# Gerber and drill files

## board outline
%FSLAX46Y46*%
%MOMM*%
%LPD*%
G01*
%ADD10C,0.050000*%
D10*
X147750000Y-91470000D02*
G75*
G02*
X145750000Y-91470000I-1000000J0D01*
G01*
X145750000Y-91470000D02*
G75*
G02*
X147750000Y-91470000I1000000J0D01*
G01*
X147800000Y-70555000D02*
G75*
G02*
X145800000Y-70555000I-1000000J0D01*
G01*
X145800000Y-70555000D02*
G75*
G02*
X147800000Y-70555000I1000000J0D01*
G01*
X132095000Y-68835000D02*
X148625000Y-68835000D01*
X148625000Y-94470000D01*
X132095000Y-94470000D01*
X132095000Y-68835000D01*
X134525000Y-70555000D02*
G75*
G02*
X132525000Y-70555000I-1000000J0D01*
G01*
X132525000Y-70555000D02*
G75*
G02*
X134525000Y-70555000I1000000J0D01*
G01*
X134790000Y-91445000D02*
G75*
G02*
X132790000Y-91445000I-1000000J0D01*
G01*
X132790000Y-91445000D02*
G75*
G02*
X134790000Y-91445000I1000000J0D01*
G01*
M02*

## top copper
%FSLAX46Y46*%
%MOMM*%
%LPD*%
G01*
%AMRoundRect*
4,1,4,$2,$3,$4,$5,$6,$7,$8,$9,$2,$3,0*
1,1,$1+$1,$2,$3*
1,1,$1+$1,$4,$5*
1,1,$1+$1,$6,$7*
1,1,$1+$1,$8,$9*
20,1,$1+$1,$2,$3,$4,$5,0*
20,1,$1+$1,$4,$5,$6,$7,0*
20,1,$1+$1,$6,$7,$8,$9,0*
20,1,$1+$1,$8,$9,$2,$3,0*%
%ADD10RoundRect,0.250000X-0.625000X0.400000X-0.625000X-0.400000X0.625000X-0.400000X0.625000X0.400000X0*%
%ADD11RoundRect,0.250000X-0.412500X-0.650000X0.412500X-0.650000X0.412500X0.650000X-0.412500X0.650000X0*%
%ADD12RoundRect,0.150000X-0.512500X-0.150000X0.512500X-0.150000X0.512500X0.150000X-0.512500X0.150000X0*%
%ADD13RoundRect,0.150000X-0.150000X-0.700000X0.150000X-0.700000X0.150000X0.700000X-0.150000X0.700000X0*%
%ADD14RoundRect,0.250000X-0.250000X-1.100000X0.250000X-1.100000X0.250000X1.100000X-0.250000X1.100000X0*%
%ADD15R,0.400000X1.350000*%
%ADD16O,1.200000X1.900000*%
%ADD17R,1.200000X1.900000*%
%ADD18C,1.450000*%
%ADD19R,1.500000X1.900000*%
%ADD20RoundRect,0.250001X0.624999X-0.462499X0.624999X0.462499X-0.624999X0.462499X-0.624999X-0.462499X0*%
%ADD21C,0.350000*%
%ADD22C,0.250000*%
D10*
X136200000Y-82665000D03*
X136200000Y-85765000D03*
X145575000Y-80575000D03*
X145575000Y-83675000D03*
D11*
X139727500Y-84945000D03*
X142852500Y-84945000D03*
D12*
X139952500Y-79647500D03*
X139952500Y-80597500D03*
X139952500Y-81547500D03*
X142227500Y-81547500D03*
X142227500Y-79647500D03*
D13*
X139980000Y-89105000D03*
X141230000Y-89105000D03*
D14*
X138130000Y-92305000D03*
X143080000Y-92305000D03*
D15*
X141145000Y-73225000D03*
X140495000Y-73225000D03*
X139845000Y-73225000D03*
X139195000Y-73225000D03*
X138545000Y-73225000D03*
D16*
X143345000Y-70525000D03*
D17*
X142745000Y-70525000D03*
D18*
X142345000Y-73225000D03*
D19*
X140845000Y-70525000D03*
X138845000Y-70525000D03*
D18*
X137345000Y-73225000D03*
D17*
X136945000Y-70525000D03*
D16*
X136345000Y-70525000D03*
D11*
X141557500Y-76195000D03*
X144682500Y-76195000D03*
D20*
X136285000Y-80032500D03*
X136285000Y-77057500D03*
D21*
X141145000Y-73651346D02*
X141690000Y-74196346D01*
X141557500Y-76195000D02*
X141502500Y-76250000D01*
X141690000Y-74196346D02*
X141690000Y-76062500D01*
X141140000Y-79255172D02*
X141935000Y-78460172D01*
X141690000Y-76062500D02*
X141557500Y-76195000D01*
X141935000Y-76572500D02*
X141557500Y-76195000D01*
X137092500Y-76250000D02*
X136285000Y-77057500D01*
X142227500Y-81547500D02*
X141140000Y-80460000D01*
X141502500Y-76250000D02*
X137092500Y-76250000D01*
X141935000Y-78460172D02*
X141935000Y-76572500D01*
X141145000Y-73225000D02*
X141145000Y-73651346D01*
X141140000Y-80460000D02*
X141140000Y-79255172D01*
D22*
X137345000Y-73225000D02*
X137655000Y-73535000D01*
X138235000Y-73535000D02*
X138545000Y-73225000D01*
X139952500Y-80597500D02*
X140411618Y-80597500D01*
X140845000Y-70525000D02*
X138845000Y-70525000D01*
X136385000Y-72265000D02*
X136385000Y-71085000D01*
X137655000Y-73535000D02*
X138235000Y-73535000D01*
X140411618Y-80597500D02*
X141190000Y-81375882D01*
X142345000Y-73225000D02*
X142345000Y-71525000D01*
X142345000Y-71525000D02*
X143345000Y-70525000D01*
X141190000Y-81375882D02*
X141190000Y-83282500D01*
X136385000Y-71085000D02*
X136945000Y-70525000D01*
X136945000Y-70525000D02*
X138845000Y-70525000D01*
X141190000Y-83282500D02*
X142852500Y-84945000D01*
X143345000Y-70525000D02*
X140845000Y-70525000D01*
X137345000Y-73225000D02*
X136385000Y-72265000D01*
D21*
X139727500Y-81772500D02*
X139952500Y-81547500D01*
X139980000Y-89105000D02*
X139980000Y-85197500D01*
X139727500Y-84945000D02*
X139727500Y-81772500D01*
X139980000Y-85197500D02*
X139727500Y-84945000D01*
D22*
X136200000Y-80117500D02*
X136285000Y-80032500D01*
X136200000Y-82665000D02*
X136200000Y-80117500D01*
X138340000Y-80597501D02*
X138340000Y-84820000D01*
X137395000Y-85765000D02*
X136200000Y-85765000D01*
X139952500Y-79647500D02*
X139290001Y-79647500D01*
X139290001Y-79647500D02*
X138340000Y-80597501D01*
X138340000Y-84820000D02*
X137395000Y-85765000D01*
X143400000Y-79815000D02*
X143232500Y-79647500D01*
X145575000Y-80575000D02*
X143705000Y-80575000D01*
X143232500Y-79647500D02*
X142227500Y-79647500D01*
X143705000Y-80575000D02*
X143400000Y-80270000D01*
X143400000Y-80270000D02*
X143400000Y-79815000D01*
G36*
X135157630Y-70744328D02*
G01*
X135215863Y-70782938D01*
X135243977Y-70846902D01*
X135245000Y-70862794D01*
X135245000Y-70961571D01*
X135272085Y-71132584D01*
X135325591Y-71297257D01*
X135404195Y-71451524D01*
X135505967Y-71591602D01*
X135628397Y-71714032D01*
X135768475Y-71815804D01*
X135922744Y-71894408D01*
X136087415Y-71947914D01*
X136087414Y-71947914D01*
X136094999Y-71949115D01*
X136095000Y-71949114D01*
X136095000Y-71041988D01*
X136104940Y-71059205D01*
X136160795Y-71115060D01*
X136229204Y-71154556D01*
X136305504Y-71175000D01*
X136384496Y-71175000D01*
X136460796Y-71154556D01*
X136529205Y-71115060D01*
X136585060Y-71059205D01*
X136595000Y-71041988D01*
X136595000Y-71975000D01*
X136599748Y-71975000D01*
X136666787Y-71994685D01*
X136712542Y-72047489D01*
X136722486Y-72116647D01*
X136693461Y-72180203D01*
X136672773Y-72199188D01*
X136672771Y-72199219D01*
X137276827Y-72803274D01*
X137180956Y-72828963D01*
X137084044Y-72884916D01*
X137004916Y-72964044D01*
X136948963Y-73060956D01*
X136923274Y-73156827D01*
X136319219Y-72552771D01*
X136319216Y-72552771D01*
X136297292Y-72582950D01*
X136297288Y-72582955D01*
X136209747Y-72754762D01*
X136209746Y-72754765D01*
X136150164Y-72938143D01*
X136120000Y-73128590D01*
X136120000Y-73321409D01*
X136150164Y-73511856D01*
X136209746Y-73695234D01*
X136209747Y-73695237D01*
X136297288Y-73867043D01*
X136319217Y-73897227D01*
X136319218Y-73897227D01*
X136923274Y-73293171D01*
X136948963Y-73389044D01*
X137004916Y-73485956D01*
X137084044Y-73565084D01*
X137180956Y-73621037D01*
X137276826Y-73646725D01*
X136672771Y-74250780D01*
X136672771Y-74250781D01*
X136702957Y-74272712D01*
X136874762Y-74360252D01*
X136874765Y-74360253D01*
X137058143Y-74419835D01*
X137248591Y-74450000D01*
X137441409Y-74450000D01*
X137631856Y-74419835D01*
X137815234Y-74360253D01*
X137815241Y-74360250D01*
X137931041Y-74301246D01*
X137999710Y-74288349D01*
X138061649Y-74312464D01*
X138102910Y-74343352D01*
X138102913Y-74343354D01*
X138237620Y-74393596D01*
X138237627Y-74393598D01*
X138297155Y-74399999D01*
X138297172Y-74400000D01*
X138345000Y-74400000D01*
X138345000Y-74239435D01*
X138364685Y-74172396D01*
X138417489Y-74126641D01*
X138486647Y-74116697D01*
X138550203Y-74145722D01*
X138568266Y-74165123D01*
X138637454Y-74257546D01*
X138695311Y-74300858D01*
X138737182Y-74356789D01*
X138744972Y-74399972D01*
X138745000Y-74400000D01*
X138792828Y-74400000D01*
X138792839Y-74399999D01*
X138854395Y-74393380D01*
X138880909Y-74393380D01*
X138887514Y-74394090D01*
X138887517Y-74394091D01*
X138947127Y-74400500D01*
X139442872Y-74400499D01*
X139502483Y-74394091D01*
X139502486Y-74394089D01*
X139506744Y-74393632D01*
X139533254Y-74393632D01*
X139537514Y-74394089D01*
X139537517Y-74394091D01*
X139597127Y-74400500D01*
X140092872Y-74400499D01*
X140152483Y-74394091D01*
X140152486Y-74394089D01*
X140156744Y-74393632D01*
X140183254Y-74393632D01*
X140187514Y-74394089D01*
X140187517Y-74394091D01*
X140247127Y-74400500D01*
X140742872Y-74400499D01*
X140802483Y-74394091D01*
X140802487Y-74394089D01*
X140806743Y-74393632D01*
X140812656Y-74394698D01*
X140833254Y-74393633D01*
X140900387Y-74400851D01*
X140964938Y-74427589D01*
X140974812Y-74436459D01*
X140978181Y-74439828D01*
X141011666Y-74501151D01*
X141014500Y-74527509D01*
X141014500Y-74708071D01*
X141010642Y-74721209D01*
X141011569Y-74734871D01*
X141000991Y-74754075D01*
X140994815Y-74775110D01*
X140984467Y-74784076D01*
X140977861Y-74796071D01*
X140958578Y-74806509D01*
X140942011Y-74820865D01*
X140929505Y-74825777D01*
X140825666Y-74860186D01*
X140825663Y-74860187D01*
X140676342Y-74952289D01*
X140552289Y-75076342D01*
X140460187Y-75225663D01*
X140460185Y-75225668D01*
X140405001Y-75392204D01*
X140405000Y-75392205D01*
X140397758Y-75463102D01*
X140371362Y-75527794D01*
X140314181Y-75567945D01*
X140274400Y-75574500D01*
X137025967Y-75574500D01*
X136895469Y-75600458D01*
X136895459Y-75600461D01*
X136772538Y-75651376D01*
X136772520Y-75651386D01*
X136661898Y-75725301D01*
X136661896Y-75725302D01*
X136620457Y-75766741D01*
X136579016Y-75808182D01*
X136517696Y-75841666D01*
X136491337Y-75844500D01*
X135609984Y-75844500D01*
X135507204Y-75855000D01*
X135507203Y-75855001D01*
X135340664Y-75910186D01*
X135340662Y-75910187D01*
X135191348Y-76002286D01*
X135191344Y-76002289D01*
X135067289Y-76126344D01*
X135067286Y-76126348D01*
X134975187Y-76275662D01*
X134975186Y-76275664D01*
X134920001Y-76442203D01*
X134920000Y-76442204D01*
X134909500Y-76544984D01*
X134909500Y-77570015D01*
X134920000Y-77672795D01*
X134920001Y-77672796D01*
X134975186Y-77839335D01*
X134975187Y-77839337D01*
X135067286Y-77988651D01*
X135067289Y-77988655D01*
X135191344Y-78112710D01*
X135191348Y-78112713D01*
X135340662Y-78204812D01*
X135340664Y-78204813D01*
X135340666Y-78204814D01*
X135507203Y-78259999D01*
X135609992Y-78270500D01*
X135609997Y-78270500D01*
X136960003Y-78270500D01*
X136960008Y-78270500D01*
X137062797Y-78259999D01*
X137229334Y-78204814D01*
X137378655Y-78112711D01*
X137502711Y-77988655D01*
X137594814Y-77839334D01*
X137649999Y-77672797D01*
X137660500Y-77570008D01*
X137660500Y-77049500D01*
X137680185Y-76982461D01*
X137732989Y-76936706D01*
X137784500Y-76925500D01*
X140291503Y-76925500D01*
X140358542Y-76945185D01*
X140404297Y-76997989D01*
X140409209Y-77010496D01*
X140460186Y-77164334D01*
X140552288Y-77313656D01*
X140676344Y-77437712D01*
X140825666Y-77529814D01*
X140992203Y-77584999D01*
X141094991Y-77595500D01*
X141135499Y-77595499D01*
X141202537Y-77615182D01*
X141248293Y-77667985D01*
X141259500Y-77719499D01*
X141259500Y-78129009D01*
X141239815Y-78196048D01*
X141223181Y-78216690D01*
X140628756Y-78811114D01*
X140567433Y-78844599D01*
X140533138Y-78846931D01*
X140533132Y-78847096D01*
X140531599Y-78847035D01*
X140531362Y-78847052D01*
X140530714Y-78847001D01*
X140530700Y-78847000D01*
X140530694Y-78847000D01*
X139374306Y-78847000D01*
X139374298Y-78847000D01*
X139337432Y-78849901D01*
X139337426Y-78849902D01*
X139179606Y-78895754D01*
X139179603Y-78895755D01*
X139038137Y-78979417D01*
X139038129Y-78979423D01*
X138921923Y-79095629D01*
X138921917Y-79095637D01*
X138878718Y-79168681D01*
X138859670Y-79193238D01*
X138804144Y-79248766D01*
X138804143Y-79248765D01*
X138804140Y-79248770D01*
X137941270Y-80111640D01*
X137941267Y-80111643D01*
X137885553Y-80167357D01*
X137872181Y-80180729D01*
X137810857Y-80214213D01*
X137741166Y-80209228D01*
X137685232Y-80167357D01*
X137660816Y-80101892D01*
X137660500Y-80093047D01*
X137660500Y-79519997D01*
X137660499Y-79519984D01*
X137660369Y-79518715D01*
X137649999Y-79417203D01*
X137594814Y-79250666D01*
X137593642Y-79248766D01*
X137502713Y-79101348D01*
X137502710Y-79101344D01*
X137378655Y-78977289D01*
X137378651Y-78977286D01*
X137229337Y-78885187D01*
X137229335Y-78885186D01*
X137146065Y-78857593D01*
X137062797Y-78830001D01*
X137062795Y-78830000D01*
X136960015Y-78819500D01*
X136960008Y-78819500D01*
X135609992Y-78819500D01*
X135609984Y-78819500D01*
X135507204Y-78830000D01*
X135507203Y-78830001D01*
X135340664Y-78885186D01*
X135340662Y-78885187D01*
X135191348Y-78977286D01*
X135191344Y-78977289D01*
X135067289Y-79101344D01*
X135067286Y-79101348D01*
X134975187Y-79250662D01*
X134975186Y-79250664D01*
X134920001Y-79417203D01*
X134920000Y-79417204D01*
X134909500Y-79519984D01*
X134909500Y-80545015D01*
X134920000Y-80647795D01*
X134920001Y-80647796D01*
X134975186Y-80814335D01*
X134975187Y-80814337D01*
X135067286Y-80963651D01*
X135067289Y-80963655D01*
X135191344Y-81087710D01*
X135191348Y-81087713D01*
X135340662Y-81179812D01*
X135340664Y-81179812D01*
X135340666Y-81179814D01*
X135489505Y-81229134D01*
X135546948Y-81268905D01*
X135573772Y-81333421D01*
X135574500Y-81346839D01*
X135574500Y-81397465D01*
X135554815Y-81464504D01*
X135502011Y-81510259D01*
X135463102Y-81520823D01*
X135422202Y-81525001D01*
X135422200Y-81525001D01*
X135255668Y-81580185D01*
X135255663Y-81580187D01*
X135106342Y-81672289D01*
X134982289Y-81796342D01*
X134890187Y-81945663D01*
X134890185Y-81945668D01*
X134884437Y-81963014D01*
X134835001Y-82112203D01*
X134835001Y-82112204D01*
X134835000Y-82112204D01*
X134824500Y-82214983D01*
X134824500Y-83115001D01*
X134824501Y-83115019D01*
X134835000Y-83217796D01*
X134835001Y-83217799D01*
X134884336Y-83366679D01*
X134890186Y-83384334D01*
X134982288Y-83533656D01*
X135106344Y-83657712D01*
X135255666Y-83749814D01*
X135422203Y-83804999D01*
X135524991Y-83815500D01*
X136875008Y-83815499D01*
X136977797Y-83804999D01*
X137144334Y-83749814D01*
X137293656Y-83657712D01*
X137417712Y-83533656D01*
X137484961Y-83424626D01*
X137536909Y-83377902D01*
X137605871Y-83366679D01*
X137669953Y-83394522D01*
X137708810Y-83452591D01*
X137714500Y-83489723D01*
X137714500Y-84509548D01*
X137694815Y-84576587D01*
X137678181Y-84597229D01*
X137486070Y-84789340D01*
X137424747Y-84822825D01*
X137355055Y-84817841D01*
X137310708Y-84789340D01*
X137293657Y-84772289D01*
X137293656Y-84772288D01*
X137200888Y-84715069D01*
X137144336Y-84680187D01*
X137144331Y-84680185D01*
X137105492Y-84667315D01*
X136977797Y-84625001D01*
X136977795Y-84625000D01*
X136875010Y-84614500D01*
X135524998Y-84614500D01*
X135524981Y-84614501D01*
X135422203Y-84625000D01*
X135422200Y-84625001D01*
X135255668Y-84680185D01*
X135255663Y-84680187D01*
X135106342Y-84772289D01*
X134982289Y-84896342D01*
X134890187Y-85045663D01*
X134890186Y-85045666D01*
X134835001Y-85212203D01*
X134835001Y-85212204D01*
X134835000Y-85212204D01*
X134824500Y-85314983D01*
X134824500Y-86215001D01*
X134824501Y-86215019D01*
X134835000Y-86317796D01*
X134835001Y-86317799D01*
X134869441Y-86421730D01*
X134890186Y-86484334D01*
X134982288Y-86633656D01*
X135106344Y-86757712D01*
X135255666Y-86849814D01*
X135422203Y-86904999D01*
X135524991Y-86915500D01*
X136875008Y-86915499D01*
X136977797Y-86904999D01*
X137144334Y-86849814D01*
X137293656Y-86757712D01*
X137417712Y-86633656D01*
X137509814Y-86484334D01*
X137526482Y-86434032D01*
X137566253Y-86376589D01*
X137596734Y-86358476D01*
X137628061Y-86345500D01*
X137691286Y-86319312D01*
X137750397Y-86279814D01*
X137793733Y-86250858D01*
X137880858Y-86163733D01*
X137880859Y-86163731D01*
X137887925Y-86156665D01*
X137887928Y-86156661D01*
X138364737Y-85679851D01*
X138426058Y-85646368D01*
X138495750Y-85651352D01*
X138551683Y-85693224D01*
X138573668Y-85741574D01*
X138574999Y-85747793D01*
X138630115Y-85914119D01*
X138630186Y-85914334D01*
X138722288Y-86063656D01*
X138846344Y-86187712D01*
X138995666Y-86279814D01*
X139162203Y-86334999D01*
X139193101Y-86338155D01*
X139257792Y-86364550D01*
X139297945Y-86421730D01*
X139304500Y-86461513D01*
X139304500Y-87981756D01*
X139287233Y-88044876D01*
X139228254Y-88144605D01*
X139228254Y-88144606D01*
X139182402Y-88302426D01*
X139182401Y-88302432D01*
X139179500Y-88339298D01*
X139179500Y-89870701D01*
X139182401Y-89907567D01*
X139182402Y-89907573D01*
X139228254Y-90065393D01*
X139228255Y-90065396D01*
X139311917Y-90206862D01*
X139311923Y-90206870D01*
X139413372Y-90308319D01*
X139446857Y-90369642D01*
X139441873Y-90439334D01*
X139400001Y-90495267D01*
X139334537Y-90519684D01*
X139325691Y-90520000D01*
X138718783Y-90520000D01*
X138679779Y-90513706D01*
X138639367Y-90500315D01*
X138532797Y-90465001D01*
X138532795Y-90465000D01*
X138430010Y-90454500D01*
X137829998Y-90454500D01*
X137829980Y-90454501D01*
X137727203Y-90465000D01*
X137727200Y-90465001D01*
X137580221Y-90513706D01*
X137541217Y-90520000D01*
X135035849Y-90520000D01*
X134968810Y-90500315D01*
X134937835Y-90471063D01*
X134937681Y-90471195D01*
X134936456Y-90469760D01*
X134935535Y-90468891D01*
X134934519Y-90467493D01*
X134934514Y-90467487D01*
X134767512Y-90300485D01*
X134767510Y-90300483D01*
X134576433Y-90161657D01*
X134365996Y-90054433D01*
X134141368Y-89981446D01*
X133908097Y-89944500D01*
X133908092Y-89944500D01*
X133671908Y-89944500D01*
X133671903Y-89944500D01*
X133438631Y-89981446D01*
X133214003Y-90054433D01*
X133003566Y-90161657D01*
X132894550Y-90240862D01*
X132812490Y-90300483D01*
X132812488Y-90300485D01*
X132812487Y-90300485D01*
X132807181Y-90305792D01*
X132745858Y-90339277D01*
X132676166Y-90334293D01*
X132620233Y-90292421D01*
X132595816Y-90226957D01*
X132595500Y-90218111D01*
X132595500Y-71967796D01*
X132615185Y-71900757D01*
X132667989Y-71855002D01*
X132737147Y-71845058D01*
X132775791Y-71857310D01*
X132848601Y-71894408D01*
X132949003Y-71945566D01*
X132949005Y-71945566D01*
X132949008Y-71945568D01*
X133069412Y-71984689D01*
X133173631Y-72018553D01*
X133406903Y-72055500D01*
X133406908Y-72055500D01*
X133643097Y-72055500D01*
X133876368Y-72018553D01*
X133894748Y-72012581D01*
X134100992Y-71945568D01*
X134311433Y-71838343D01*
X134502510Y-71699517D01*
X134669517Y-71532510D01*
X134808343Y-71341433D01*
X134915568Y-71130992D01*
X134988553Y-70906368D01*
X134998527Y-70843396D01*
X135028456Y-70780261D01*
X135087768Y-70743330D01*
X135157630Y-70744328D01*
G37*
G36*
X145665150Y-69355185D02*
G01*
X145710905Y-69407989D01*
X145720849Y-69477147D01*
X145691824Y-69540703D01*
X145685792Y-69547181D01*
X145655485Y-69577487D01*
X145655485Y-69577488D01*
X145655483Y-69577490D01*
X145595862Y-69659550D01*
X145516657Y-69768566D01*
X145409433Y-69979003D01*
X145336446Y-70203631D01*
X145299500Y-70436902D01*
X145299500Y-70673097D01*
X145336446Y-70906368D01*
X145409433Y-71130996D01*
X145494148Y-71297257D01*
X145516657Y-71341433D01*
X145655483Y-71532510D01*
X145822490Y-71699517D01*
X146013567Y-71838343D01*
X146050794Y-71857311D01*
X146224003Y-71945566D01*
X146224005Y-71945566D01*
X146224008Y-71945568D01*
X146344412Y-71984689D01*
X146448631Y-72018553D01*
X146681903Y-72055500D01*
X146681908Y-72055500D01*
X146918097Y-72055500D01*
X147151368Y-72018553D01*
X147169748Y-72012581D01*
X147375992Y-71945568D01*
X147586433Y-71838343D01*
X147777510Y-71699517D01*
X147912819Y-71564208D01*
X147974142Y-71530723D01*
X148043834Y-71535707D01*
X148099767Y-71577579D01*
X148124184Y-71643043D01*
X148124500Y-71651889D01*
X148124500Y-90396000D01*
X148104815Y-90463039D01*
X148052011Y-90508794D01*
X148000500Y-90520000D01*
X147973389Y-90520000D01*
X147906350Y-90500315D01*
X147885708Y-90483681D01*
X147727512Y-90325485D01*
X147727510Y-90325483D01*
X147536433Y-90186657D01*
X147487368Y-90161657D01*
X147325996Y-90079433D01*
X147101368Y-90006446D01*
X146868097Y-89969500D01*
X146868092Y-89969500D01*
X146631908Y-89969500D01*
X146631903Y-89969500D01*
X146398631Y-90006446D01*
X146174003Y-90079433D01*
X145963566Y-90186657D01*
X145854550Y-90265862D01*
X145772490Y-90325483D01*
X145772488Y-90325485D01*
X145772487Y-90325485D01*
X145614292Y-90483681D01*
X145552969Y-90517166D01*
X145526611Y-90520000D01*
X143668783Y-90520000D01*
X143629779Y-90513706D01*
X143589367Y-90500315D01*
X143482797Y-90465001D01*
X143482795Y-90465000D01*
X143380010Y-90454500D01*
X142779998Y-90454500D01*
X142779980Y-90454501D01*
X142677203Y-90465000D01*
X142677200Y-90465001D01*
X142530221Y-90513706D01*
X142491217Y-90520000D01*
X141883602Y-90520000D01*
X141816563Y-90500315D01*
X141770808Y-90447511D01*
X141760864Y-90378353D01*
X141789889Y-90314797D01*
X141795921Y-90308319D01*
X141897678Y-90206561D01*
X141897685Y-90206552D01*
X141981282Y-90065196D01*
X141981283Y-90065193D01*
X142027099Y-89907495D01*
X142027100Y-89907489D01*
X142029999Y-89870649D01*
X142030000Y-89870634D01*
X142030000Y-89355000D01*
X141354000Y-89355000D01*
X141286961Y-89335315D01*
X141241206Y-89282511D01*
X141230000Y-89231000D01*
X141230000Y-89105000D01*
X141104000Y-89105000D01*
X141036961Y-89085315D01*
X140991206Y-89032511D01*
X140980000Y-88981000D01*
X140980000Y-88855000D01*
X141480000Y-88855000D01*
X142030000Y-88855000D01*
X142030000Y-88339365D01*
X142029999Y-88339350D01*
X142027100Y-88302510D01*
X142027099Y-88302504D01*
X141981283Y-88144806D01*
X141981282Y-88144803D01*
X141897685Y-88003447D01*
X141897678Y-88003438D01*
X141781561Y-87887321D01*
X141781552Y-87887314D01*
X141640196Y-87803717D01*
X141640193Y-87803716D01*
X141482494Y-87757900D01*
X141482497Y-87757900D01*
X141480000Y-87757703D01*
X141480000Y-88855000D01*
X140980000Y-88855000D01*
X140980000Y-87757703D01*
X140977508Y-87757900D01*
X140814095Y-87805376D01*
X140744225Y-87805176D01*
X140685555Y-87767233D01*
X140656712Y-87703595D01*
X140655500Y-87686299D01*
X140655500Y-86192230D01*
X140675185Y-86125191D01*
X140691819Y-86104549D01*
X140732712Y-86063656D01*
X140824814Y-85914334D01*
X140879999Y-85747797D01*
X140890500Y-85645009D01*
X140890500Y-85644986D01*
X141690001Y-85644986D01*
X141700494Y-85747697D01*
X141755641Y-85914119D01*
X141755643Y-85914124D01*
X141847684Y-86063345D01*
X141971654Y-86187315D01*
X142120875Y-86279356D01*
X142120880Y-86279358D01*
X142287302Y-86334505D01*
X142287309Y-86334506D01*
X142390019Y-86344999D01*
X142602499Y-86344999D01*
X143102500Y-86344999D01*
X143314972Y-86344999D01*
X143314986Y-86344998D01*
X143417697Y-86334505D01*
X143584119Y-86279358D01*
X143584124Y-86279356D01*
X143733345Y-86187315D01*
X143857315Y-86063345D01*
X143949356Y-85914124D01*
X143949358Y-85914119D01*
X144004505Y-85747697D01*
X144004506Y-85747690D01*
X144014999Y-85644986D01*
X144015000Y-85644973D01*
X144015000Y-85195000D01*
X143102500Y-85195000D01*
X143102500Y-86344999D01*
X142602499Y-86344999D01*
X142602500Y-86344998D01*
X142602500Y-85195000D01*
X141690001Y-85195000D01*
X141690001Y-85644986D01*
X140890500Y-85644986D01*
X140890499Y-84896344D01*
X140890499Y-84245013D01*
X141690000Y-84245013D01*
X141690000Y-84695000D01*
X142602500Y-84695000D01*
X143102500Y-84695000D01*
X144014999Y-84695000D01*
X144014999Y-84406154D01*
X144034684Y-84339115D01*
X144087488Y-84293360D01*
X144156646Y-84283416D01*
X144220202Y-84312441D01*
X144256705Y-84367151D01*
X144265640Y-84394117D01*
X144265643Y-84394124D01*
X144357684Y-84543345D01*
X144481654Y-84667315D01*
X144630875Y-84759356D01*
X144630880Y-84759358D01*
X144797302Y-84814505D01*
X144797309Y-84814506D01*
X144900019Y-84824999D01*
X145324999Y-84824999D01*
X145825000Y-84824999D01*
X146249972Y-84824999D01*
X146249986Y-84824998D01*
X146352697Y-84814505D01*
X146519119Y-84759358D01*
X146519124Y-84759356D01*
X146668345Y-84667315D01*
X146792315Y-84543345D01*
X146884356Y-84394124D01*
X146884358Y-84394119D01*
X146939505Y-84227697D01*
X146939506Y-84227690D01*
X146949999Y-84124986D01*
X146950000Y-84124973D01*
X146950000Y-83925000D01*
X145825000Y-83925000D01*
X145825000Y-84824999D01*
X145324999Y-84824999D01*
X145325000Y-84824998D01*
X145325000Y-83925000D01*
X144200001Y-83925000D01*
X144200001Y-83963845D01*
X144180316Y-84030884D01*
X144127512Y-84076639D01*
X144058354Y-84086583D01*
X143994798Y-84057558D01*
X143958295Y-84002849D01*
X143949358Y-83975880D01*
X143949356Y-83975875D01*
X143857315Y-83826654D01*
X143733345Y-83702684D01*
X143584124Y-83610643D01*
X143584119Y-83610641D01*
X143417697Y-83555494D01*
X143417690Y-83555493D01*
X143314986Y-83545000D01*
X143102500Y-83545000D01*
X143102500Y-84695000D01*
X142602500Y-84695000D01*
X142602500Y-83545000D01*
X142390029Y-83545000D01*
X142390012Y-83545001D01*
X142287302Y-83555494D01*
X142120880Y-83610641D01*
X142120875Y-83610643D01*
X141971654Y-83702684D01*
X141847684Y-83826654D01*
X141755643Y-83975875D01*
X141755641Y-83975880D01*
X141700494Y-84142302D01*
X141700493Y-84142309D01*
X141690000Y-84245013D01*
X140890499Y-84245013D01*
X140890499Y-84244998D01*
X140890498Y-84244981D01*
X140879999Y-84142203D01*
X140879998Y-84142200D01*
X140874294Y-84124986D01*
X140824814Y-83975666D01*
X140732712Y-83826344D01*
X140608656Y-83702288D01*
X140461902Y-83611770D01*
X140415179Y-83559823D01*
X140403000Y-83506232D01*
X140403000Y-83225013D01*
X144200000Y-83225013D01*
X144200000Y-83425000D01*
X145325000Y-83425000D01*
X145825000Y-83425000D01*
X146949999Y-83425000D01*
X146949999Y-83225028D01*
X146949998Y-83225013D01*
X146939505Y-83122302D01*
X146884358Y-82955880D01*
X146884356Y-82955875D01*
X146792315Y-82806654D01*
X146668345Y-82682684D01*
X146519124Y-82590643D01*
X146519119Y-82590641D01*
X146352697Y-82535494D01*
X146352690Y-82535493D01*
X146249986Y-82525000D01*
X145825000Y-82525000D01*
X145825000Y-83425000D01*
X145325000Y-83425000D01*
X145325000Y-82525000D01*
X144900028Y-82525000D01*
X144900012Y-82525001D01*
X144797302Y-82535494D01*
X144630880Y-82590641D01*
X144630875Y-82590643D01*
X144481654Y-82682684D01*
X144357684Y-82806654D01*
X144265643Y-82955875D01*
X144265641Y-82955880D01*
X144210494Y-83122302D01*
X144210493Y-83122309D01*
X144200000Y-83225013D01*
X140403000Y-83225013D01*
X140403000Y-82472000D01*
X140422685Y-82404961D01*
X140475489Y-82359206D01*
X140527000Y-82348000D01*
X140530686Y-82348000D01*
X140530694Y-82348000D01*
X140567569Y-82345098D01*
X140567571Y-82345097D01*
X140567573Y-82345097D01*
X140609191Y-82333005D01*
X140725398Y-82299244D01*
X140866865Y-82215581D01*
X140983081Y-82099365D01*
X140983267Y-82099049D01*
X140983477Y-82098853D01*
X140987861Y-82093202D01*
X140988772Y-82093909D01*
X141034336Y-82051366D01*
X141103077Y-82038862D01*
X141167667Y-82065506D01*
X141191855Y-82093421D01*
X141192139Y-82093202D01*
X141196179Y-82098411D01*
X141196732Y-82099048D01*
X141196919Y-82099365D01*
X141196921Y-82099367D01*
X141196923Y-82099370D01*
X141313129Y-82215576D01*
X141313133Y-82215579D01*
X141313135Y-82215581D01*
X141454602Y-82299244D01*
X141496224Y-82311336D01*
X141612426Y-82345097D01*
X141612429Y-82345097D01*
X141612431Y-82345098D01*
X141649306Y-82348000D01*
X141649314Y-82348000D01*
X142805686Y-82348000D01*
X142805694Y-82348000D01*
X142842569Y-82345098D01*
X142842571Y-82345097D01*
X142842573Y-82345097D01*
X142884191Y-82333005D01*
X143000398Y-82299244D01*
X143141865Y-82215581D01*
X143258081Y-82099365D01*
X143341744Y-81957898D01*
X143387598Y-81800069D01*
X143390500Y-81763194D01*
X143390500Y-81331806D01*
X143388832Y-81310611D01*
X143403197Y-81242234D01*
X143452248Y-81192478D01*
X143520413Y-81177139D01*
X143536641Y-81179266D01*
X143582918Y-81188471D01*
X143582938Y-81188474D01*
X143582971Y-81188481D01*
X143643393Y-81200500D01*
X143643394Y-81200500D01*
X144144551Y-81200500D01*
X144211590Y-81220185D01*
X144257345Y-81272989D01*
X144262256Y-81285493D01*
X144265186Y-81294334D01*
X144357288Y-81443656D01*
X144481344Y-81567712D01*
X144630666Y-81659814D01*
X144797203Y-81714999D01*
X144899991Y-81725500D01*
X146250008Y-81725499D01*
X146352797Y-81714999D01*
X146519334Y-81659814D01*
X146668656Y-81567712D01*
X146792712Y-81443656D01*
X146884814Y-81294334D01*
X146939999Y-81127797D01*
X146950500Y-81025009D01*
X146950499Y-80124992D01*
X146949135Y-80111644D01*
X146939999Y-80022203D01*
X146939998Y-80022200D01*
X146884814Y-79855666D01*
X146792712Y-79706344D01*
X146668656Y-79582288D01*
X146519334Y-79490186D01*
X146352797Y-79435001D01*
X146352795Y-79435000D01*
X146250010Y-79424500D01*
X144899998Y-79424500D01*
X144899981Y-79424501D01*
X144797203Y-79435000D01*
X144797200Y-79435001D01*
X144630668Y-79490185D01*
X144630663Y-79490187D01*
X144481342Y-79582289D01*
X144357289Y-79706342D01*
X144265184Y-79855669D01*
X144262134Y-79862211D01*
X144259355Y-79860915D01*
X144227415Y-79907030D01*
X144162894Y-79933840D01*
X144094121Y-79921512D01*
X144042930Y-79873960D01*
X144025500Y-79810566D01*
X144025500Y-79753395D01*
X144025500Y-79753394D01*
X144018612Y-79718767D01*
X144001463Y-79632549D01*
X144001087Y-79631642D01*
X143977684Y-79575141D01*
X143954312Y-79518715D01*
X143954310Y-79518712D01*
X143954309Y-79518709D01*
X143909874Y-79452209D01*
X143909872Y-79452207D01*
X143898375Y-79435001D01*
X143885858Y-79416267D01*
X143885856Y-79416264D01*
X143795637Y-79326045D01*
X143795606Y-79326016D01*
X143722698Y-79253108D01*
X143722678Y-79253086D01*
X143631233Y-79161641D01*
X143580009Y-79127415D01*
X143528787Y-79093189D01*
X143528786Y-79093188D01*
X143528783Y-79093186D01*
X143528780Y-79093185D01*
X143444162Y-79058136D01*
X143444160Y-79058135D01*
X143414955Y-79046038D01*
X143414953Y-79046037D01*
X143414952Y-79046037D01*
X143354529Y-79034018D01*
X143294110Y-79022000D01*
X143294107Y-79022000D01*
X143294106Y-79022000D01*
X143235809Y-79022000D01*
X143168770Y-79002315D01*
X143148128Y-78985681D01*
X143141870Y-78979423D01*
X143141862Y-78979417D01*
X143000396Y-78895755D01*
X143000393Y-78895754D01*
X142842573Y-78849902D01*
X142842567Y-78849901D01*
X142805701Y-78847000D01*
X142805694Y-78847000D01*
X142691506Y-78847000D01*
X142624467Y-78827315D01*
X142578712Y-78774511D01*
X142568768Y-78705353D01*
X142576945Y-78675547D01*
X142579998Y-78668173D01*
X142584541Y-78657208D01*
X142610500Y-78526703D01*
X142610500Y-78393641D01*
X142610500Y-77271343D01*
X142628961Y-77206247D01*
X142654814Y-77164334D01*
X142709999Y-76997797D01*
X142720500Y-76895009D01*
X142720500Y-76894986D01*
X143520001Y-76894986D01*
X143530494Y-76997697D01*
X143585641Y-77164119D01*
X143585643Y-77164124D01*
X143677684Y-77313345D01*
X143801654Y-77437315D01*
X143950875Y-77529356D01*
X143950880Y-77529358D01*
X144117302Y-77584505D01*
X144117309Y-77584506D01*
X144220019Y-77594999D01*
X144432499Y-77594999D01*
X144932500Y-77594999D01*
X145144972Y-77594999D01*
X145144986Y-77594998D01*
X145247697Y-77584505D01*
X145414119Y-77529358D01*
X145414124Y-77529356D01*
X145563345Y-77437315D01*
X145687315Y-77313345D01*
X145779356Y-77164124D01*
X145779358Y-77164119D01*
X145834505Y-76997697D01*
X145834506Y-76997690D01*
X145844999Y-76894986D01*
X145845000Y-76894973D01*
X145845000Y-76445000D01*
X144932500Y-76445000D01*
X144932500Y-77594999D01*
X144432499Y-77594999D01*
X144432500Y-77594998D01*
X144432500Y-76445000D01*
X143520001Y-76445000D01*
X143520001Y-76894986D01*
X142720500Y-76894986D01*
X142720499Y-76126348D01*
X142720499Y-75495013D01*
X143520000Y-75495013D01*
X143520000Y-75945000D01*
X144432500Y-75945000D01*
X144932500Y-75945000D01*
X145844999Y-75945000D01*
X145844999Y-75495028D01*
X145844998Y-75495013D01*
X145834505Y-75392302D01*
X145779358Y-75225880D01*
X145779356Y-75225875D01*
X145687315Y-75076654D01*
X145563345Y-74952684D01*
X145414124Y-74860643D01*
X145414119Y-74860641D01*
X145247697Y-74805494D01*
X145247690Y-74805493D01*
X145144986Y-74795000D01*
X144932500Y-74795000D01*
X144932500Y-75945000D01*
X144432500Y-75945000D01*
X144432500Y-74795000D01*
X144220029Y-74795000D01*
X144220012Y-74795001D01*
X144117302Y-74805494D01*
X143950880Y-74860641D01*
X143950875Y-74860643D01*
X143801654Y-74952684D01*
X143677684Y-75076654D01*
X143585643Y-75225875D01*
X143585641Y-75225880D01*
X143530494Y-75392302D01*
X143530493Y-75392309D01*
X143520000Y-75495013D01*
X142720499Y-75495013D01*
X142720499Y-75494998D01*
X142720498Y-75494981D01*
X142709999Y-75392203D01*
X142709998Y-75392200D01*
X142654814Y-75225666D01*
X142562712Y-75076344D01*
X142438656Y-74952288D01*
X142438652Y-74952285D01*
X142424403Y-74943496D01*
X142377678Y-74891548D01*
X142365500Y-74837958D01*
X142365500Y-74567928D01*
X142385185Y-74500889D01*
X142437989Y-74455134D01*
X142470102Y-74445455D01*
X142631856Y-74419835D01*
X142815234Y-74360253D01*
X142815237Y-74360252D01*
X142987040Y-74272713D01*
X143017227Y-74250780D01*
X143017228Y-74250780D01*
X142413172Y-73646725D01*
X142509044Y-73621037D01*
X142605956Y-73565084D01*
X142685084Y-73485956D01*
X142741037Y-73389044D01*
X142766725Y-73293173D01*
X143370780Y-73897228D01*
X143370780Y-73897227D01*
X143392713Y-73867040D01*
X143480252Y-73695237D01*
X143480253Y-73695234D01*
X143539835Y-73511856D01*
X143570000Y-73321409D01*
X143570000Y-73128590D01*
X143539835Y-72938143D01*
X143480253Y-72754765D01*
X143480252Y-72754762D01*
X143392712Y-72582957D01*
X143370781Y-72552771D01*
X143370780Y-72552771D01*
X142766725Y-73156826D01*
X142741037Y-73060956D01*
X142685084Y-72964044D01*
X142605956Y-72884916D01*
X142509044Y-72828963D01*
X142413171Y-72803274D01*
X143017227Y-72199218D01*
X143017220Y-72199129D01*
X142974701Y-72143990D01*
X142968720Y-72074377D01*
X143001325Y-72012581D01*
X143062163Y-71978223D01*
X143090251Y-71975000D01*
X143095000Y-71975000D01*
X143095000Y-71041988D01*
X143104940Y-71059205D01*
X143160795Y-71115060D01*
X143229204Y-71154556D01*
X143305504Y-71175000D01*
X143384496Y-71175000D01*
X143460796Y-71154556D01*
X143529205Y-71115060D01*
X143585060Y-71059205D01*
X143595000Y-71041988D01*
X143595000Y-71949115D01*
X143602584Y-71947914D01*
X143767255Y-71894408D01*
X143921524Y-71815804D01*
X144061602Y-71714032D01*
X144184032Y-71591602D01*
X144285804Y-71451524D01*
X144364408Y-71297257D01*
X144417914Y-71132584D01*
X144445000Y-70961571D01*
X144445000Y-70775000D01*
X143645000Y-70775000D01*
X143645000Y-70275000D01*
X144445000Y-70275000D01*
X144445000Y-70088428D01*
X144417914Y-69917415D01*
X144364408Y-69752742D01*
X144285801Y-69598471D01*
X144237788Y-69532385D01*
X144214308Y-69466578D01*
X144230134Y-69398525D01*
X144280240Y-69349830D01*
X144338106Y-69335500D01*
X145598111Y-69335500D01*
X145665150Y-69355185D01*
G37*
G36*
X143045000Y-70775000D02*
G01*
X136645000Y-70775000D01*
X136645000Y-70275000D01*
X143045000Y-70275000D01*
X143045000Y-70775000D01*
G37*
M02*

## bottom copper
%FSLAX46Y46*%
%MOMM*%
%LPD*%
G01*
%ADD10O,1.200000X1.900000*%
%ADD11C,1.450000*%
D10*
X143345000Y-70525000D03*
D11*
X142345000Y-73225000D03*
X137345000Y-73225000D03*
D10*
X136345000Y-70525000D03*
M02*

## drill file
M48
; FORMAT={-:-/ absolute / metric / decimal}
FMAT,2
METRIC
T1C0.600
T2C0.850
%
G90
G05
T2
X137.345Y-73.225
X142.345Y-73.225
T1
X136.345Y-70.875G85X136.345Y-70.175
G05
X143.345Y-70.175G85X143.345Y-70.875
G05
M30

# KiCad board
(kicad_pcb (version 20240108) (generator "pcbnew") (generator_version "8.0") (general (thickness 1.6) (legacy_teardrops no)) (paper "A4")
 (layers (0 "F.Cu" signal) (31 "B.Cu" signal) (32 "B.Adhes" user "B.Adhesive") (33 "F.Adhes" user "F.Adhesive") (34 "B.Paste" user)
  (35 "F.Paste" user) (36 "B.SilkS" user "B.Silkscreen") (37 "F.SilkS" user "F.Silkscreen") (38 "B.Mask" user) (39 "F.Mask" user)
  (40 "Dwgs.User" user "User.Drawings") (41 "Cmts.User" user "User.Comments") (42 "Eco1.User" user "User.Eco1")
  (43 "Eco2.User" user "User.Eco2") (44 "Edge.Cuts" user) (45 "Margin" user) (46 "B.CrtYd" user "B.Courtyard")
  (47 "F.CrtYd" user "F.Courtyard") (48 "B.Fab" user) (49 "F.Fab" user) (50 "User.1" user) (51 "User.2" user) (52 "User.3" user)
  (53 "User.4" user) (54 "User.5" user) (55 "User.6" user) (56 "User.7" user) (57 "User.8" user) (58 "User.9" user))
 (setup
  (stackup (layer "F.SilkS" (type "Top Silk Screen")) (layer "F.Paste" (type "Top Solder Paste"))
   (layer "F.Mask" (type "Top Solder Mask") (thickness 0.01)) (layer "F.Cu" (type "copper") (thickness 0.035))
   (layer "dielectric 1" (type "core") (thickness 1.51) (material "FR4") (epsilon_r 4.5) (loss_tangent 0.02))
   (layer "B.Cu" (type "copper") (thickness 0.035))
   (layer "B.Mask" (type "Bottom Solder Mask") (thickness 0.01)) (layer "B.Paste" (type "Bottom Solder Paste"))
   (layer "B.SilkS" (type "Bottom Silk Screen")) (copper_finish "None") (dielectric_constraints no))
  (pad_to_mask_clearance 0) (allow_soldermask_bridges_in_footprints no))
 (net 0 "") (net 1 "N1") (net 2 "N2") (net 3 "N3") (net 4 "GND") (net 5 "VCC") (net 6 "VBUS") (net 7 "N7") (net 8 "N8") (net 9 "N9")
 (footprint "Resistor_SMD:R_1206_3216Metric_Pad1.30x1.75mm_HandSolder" (layer "F.Cu") (at 136.2 84.215 -90)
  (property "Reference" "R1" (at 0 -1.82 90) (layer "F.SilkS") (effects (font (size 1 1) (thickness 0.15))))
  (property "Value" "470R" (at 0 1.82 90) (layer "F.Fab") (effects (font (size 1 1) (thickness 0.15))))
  (pad "1" smd roundrect (at -1.55 0 270) (size 1.3 1.75) (layers "F.Cu" "F.Paste" "F.Mask") (roundrect_rratio 0.192308) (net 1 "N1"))
  (pad "2" smd roundrect (at 1.55 0 270) (size 1.3 1.75) (layers "F.Cu" "F.Paste" "F.Mask") (roundrect_rratio 0.192308) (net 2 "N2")))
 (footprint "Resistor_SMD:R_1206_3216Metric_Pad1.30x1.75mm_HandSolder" (layer "F.Cu") (at 145.575 82.125 -90)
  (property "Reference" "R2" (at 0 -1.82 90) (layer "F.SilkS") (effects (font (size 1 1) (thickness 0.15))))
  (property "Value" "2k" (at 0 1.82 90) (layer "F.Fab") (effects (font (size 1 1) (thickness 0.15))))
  (pad "1" smd roundrect (at -1.55 0 270) (size 1.3 1.75) (layers "F.Cu" "F.Paste" "F.Mask") (roundrect_rratio 0.192308) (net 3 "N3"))
  (pad "2" smd roundrect (at 1.55 0 270) (size 1.3 1.75) (layers "F.Cu" "F.Paste" "F.Mask") (roundrect_rratio 0.192308) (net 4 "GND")))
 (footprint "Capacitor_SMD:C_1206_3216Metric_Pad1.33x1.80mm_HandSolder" (layer "F.Cu") (at 141.29 84.945)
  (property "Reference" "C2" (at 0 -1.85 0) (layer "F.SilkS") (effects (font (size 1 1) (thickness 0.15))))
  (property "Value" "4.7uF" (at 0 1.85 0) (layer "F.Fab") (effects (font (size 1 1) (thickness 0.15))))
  (pad "1" smd roundrect (at -1.5625 0) (size 1.325 1.8) (layers "F.Cu" "F.Paste" "F.Mask") (roundrect_rratio 0.188679) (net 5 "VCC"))
  (pad "2" smd roundrect (at 1.5625 0) (size 1.325 1.8) (layers "F.Cu" "F.Paste" "F.Mask") (roundrect_rratio 0.188679) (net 4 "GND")))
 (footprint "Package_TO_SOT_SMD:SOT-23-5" (layer "F.Cu") (at 141.09 80.5975)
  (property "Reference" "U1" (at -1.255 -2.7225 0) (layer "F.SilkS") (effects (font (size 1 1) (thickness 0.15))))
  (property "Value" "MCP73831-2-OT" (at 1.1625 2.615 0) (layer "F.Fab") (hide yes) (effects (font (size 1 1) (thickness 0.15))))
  (pad "1" smd roundrect (at -1.1375 -0.95) (size 1.325 0.6) (layers "F.Cu" "F.Paste" "F.Mask") (roundrect_rratio 0.25) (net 2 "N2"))
  (pad "2" smd roundrect (at -1.1375 0) (size 1.325 0.6) (layers "F.Cu" "F.Paste" "F.Mask") (roundrect_rratio 0.25) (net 4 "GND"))
  (pad "3" smd roundrect (at -1.1375 0.95) (size 1.325 0.6) (layers "F.Cu" "F.Paste" "F.Mask") (roundrect_rratio 0.25) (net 5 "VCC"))
  (pad "4" smd roundrect (at 1.1375 0.95) (size 1.325 0.6) (layers "F.Cu" "F.Paste" "F.Mask") (roundrect_rratio 0.25) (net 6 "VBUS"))
  (pad "5" smd roundrect (at 1.1375 -0.95) (size 1.325 0.6) (layers "F.Cu" "F.Paste" "F.Mask") (roundrect_rratio 0.25) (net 3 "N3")))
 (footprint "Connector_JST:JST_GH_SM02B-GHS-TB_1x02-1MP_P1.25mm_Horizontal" (layer "F.Cu") (at 140.605 90.955)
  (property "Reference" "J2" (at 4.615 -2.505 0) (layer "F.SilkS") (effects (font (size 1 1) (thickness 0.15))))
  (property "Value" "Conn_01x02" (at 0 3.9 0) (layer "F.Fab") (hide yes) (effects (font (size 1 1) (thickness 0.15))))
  (pad "1" smd roundrect (at -0.625 -1.85) (size 0.6 1.7) (layers "F.Cu" "F.Paste" "F.Mask") (roundrect_rratio 0.25) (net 5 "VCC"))
  (pad "2" smd roundrect (at 0.625 -1.85) (size 0.6 1.7) (layers "F.Cu" "F.Paste" "F.Mask") (roundrect_rratio 0.25) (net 4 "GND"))
  (pad "MP" smd roundrect (at -2.475 1.35) (size 1 2.7) (layers "F.Cu" "F.Paste" "F.Mask") (roundrect_rratio 0.25))
  (pad "MP" smd roundrect (at 2.475 1.35) (size 1 2.7) (layers "F.Cu" "F.Paste" "F.Mask") (roundrect_rratio 0.25)))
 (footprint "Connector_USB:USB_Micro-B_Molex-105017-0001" (layer "F.Cu") (at 139.845 71.7625 180)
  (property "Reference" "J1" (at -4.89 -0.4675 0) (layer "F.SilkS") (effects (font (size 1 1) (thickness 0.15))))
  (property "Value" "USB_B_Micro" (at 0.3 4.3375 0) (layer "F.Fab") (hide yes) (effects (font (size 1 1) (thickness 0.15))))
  (pad "1" smd rect (at -1.3 -1.4625 180) (size 0.4 1.35) (layers "F.Cu" "F.Paste" "F.Mask") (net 6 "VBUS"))
  (pad "2" smd rect (at -0.65 -1.4625 180) (size 0.4 1.35) (layers "F.Cu" "F.Paste" "F.Mask") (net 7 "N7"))
  (pad "3" smd rect (at 0 -1.4625 180) (size 0.4 1.35) (layers "F.Cu" "F.Paste" "F.Mask") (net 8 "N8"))
  (pad "4" smd rect (at 0.65 -1.4625 180) (size 0.4 1.35) (layers "F.Cu" "F.Paste" "F.Mask") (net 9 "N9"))
  (pad "5" smd rect (at 1.3 -1.4625 180) (size 0.4 1.35) (layers "F.Cu" "F.Paste" "F.Mask") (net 4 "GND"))
  (pad "6" thru_hole oval (at -3.5 1.2375) (size 1.2 1.9) (drill oval 0.6 1.3) (layers "*.Cu" "*.Mask") (remove_unused_layers no)
   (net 4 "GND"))
  (pad "6" smd rect (at -2.9 1.2375 180) (size 1.2 1.9) (layers "F.Cu" "F.Mask") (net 4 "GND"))
  (pad "6" thru_hole circle (at -2.5 -1.4625 180) (size 1.45 1.45) (drill 0.85) (layers "*.Cu" "*.Mask") (remove_unused_layers no)
   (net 4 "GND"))
  (pad "6" smd rect (at -1 1.2375 180) (size 1.5 1.9) (layers "F.Cu" "F.Paste" "F.Mask") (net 4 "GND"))
  (pad "6" smd rect (at 1 1.2375 180) (size 1.5 1.9) (layers "F.Cu" "F.Paste" "F.Mask") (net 4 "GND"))
  (pad "6" thru_hole circle (at 2.5 -1.4625 180) (size 1.45 1.45) (drill 0.85) (layers "*.Cu" "*.Mask") (remove_unused_layers no)
   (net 4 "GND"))
  (pad "6" smd rect (at 2.9 1.2375 180) (size 1.2 1.9) (layers "F.Cu" "F.Mask") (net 4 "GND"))
  (pad "6" thru_hole oval (at 3.5 1.2375 180) (size 1.2 1.9) (drill oval 0.6 1.3) (layers "*.Cu" "*.Mask") (remove_unused_layers no)
   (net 4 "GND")))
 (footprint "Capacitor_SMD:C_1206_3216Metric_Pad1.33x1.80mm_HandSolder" (layer "F.Cu") (at 143.12 76.195)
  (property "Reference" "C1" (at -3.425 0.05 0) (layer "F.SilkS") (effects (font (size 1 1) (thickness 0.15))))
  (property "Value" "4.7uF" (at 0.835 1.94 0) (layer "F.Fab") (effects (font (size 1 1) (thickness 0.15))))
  (pad "1" smd roundrect (at -1.5625 0) (size 1.325 1.8) (layers "F.Cu" "F.Paste" "F.Mask") (roundrect_rratio 0.188679) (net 6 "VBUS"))
  (pad "2" smd roundrect (at 1.5625 0) (size 1.325 1.8) (layers "F.Cu" "F.Paste" "F.Mask") (roundrect_rratio 0.188679) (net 4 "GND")))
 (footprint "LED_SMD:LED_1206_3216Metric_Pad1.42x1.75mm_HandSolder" (layer "F.Cu") (at 136.285 78.545 90)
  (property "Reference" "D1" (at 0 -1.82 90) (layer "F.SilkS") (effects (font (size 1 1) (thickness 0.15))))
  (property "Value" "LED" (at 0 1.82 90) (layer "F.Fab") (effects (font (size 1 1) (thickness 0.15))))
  (pad "1" smd roundrect (at -1.4875 0 90) (size 1.425 1.75) (layers "F.Cu" "F.Paste" "F.Mask") (roundrect_rratio 0.175439) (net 1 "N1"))
  (pad "2" smd roundrect (at 1.4875 0 90) (size 1.425 1.75) (layers "F.Cu" "F.Paste" "F.Mask") (roundrect_rratio 0.175439) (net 6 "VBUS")))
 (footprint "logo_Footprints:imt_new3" (layer "B.Cu") (at 139.655 81.51 90)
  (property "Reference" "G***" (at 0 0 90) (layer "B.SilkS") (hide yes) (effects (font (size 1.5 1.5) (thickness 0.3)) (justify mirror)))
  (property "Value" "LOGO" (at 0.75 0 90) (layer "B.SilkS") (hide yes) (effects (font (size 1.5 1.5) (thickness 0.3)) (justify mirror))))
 (gr_circle (center 146.75 91.47) (end 147.75 91.47) (stroke (width 0.05) (type default)) (fill none) (layer "Edge.Cuts"))
 (gr_circle (center 146.8 70.555) (end 147.8 70.555) (stroke (width 0.05) (type default)) (fill none) (layer "Edge.Cuts"))
 (gr_rect (start 132.095 68.835) (end 148.625 94.47) (stroke (width 0.05) (type default)) (fill none) (layer "Edge.Cuts"))
 (gr_circle (center 133.525 70.555) (end 134.525 70.555) (stroke (width 0.05) (type default)) (fill none) (layer "Edge.Cuts"))
 (gr_circle (center 133.79 91.445) (end 134.79 91.445) (stroke (width 0.05) (type default)) (fill none) (layer "Edge.Cuts"))
 (segment (start 141.145 73.651346) (end 141.69 74.196346) (width 0.35) (layer "F.Cu") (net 6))
 (segment (start 141.5575 76.195) (end 141.5025 76.25) (width 0.35) (layer "F.Cu") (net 6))
 (segment (start 141.69 74.196346) (end 141.69 76.0625) (width 0.35) (layer "F.Cu") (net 6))
 (segment (start 141.14 79.255172) (end 141.935 78.460172) (width 0.35) (layer "F.Cu") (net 6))
 (segment (start 141.69 76.0625) (end 141.5575 76.195) (width 0.35) (layer "F.Cu") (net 6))
 (segment (start 141.935 76.5725) (end 141.5575 76.195) (width 0.35) (layer "F.Cu") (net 6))
 (segment (start 137.0925 76.25) (end 136.285 77.0575) (width 0.35) (layer "F.Cu") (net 6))
 (segment (start 142.2275 81.5475) (end 141.14 80.46) (width 0.35) (layer "F.Cu") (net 6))
 (segment (start 141.5025 76.25) (end 137.0925 76.25) (width 0.35) (layer "F.Cu") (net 6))
 (segment (start 141.935 78.460172) (end 141.935 76.5725) (width 0.35) (layer "F.Cu") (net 6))
 (segment (start 141.145 73.225) (end 141.145 73.651346) (width 0.35) (layer "F.Cu") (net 6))
 (segment (start 141.14 80.46) (end 141.14 79.255172) (width 0.35) (layer "F.Cu") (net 6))
 (segment (start 137.345 73.225) (end 137.655 73.535) (width 0.25) (layer "F.Cu") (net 4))
 (segment (start 138.235 73.535) (end 138.545 73.225) (width 0.25) (layer "F.Cu") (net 4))
 (segment (start 139.9525 80.5975) (end 140.411618 80.5975) (width 0.25) (layer "F.Cu") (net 4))
 (segment (start 140.845 70.525) (end 138.845 70.525) (width 0.25) (layer "F.Cu") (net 4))
 (segment (start 136.385 72.265) (end 136.385 71.085) (width 0.25) (layer "F.Cu") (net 4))
 (segment (start 137.655 73.535) (end 138.235 73.535) (width 0.25) (layer "F.Cu") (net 4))
 (segment (start 140.411618 80.5975) (end 141.19 81.375882) (width 0.25) (layer "F.Cu") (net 4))
 (segment (start 142.345 73.225) (end 142.345 71.525) (width 0.25) (layer "F.Cu") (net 4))
 (segment (start 142.345 71.525) (end 143.345 70.525) (width 0.25) (layer "F.Cu") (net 4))
 (segment (start 141.19 81.375882) (end 141.19 83.2825) (width 0.25) (layer "F.Cu") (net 4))
 (segment (start 136.385 71.085) (end 136.945 70.525) (width 0.25) (layer "F.Cu") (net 4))
 (segment (start 136.945 70.525) (end 138.845 70.525) (width 0.25) (layer "F.Cu") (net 4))
 (segment (start 141.19 83.2825) (end 142.8525 84.945) (width 0.25) (layer "F.Cu") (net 4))
 (segment (start 143.345 70.525) (end 140.845 70.525) (width 0.25) (layer "F.Cu") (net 4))
 (segment (start 137.345 73.225) (end 136.385 72.265) (width 0.25) (layer "F.Cu") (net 4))
 (segment (start 139.7275 81.7725) (end 139.9525 81.5475) (width 0.35) (layer "F.Cu") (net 5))
 (segment (start 139.98 89.105) (end 139.98 85.1975) (width 0.35) (layer "F.Cu") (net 5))
 (segment (start 139.7275 84.945) (end 139.7275 81.7725) (width 0.35) (layer "F.Cu") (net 5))
 (segment (start 139.98 85.1975) (end 139.7275 84.945) (width 0.35) (layer "F.Cu") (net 5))
 (segment (start 136.2 80.1175) (end 136.285 80.0325) (width 0.25) (layer "F.Cu") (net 1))
 (segment (start 136.2 82.665) (end 136.2 80.1175) (width 0.25) (layer "F.Cu") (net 1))
 (segment (start 138.34 80.597501) (end 138.34 84.82) (width 0.25) (layer "F.Cu") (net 2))
 (segment (start 137.395 85.765) (end 136.2 85.765) (width 0.25) (layer "F.Cu") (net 2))
 (segment (start 139.9525 79.6475) (end 139.290001 79.6475) (width 0.25) (layer "F.Cu") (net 2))
 (segment (start 139.290001 79.6475) (end 138.34 80.597501) (width 0.25) (layer "F.Cu") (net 2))
 (segment (start 138.34 84.82) (end 137.395 85.765) (width 0.25) (layer "F.Cu") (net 2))
 (segment (start 143.4 79.815) (end 143.2325 79.6475) (width 0.25) (layer "F.Cu") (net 3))
 (segment (start 145.575 80.575) (end 143.705 80.575) (width 0.25) (layer "F.Cu") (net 3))
 (segment (start 143.2325 79.6475) (end 142.2275 79.6475) (width 0.25) (layer "F.Cu") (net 3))
 (segment (start 143.705 80.575) (end 143.4 80.27) (width 0.25) (layer "F.Cu") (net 3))
 (segment (start 143.4 80.27) (end 143.4 79.815) (width 0.25) (layer "F.Cu") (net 3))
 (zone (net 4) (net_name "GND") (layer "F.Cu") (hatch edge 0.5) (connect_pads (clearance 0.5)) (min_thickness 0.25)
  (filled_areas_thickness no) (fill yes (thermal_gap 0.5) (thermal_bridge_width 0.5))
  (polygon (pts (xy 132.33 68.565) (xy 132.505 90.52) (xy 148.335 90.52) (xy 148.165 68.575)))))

